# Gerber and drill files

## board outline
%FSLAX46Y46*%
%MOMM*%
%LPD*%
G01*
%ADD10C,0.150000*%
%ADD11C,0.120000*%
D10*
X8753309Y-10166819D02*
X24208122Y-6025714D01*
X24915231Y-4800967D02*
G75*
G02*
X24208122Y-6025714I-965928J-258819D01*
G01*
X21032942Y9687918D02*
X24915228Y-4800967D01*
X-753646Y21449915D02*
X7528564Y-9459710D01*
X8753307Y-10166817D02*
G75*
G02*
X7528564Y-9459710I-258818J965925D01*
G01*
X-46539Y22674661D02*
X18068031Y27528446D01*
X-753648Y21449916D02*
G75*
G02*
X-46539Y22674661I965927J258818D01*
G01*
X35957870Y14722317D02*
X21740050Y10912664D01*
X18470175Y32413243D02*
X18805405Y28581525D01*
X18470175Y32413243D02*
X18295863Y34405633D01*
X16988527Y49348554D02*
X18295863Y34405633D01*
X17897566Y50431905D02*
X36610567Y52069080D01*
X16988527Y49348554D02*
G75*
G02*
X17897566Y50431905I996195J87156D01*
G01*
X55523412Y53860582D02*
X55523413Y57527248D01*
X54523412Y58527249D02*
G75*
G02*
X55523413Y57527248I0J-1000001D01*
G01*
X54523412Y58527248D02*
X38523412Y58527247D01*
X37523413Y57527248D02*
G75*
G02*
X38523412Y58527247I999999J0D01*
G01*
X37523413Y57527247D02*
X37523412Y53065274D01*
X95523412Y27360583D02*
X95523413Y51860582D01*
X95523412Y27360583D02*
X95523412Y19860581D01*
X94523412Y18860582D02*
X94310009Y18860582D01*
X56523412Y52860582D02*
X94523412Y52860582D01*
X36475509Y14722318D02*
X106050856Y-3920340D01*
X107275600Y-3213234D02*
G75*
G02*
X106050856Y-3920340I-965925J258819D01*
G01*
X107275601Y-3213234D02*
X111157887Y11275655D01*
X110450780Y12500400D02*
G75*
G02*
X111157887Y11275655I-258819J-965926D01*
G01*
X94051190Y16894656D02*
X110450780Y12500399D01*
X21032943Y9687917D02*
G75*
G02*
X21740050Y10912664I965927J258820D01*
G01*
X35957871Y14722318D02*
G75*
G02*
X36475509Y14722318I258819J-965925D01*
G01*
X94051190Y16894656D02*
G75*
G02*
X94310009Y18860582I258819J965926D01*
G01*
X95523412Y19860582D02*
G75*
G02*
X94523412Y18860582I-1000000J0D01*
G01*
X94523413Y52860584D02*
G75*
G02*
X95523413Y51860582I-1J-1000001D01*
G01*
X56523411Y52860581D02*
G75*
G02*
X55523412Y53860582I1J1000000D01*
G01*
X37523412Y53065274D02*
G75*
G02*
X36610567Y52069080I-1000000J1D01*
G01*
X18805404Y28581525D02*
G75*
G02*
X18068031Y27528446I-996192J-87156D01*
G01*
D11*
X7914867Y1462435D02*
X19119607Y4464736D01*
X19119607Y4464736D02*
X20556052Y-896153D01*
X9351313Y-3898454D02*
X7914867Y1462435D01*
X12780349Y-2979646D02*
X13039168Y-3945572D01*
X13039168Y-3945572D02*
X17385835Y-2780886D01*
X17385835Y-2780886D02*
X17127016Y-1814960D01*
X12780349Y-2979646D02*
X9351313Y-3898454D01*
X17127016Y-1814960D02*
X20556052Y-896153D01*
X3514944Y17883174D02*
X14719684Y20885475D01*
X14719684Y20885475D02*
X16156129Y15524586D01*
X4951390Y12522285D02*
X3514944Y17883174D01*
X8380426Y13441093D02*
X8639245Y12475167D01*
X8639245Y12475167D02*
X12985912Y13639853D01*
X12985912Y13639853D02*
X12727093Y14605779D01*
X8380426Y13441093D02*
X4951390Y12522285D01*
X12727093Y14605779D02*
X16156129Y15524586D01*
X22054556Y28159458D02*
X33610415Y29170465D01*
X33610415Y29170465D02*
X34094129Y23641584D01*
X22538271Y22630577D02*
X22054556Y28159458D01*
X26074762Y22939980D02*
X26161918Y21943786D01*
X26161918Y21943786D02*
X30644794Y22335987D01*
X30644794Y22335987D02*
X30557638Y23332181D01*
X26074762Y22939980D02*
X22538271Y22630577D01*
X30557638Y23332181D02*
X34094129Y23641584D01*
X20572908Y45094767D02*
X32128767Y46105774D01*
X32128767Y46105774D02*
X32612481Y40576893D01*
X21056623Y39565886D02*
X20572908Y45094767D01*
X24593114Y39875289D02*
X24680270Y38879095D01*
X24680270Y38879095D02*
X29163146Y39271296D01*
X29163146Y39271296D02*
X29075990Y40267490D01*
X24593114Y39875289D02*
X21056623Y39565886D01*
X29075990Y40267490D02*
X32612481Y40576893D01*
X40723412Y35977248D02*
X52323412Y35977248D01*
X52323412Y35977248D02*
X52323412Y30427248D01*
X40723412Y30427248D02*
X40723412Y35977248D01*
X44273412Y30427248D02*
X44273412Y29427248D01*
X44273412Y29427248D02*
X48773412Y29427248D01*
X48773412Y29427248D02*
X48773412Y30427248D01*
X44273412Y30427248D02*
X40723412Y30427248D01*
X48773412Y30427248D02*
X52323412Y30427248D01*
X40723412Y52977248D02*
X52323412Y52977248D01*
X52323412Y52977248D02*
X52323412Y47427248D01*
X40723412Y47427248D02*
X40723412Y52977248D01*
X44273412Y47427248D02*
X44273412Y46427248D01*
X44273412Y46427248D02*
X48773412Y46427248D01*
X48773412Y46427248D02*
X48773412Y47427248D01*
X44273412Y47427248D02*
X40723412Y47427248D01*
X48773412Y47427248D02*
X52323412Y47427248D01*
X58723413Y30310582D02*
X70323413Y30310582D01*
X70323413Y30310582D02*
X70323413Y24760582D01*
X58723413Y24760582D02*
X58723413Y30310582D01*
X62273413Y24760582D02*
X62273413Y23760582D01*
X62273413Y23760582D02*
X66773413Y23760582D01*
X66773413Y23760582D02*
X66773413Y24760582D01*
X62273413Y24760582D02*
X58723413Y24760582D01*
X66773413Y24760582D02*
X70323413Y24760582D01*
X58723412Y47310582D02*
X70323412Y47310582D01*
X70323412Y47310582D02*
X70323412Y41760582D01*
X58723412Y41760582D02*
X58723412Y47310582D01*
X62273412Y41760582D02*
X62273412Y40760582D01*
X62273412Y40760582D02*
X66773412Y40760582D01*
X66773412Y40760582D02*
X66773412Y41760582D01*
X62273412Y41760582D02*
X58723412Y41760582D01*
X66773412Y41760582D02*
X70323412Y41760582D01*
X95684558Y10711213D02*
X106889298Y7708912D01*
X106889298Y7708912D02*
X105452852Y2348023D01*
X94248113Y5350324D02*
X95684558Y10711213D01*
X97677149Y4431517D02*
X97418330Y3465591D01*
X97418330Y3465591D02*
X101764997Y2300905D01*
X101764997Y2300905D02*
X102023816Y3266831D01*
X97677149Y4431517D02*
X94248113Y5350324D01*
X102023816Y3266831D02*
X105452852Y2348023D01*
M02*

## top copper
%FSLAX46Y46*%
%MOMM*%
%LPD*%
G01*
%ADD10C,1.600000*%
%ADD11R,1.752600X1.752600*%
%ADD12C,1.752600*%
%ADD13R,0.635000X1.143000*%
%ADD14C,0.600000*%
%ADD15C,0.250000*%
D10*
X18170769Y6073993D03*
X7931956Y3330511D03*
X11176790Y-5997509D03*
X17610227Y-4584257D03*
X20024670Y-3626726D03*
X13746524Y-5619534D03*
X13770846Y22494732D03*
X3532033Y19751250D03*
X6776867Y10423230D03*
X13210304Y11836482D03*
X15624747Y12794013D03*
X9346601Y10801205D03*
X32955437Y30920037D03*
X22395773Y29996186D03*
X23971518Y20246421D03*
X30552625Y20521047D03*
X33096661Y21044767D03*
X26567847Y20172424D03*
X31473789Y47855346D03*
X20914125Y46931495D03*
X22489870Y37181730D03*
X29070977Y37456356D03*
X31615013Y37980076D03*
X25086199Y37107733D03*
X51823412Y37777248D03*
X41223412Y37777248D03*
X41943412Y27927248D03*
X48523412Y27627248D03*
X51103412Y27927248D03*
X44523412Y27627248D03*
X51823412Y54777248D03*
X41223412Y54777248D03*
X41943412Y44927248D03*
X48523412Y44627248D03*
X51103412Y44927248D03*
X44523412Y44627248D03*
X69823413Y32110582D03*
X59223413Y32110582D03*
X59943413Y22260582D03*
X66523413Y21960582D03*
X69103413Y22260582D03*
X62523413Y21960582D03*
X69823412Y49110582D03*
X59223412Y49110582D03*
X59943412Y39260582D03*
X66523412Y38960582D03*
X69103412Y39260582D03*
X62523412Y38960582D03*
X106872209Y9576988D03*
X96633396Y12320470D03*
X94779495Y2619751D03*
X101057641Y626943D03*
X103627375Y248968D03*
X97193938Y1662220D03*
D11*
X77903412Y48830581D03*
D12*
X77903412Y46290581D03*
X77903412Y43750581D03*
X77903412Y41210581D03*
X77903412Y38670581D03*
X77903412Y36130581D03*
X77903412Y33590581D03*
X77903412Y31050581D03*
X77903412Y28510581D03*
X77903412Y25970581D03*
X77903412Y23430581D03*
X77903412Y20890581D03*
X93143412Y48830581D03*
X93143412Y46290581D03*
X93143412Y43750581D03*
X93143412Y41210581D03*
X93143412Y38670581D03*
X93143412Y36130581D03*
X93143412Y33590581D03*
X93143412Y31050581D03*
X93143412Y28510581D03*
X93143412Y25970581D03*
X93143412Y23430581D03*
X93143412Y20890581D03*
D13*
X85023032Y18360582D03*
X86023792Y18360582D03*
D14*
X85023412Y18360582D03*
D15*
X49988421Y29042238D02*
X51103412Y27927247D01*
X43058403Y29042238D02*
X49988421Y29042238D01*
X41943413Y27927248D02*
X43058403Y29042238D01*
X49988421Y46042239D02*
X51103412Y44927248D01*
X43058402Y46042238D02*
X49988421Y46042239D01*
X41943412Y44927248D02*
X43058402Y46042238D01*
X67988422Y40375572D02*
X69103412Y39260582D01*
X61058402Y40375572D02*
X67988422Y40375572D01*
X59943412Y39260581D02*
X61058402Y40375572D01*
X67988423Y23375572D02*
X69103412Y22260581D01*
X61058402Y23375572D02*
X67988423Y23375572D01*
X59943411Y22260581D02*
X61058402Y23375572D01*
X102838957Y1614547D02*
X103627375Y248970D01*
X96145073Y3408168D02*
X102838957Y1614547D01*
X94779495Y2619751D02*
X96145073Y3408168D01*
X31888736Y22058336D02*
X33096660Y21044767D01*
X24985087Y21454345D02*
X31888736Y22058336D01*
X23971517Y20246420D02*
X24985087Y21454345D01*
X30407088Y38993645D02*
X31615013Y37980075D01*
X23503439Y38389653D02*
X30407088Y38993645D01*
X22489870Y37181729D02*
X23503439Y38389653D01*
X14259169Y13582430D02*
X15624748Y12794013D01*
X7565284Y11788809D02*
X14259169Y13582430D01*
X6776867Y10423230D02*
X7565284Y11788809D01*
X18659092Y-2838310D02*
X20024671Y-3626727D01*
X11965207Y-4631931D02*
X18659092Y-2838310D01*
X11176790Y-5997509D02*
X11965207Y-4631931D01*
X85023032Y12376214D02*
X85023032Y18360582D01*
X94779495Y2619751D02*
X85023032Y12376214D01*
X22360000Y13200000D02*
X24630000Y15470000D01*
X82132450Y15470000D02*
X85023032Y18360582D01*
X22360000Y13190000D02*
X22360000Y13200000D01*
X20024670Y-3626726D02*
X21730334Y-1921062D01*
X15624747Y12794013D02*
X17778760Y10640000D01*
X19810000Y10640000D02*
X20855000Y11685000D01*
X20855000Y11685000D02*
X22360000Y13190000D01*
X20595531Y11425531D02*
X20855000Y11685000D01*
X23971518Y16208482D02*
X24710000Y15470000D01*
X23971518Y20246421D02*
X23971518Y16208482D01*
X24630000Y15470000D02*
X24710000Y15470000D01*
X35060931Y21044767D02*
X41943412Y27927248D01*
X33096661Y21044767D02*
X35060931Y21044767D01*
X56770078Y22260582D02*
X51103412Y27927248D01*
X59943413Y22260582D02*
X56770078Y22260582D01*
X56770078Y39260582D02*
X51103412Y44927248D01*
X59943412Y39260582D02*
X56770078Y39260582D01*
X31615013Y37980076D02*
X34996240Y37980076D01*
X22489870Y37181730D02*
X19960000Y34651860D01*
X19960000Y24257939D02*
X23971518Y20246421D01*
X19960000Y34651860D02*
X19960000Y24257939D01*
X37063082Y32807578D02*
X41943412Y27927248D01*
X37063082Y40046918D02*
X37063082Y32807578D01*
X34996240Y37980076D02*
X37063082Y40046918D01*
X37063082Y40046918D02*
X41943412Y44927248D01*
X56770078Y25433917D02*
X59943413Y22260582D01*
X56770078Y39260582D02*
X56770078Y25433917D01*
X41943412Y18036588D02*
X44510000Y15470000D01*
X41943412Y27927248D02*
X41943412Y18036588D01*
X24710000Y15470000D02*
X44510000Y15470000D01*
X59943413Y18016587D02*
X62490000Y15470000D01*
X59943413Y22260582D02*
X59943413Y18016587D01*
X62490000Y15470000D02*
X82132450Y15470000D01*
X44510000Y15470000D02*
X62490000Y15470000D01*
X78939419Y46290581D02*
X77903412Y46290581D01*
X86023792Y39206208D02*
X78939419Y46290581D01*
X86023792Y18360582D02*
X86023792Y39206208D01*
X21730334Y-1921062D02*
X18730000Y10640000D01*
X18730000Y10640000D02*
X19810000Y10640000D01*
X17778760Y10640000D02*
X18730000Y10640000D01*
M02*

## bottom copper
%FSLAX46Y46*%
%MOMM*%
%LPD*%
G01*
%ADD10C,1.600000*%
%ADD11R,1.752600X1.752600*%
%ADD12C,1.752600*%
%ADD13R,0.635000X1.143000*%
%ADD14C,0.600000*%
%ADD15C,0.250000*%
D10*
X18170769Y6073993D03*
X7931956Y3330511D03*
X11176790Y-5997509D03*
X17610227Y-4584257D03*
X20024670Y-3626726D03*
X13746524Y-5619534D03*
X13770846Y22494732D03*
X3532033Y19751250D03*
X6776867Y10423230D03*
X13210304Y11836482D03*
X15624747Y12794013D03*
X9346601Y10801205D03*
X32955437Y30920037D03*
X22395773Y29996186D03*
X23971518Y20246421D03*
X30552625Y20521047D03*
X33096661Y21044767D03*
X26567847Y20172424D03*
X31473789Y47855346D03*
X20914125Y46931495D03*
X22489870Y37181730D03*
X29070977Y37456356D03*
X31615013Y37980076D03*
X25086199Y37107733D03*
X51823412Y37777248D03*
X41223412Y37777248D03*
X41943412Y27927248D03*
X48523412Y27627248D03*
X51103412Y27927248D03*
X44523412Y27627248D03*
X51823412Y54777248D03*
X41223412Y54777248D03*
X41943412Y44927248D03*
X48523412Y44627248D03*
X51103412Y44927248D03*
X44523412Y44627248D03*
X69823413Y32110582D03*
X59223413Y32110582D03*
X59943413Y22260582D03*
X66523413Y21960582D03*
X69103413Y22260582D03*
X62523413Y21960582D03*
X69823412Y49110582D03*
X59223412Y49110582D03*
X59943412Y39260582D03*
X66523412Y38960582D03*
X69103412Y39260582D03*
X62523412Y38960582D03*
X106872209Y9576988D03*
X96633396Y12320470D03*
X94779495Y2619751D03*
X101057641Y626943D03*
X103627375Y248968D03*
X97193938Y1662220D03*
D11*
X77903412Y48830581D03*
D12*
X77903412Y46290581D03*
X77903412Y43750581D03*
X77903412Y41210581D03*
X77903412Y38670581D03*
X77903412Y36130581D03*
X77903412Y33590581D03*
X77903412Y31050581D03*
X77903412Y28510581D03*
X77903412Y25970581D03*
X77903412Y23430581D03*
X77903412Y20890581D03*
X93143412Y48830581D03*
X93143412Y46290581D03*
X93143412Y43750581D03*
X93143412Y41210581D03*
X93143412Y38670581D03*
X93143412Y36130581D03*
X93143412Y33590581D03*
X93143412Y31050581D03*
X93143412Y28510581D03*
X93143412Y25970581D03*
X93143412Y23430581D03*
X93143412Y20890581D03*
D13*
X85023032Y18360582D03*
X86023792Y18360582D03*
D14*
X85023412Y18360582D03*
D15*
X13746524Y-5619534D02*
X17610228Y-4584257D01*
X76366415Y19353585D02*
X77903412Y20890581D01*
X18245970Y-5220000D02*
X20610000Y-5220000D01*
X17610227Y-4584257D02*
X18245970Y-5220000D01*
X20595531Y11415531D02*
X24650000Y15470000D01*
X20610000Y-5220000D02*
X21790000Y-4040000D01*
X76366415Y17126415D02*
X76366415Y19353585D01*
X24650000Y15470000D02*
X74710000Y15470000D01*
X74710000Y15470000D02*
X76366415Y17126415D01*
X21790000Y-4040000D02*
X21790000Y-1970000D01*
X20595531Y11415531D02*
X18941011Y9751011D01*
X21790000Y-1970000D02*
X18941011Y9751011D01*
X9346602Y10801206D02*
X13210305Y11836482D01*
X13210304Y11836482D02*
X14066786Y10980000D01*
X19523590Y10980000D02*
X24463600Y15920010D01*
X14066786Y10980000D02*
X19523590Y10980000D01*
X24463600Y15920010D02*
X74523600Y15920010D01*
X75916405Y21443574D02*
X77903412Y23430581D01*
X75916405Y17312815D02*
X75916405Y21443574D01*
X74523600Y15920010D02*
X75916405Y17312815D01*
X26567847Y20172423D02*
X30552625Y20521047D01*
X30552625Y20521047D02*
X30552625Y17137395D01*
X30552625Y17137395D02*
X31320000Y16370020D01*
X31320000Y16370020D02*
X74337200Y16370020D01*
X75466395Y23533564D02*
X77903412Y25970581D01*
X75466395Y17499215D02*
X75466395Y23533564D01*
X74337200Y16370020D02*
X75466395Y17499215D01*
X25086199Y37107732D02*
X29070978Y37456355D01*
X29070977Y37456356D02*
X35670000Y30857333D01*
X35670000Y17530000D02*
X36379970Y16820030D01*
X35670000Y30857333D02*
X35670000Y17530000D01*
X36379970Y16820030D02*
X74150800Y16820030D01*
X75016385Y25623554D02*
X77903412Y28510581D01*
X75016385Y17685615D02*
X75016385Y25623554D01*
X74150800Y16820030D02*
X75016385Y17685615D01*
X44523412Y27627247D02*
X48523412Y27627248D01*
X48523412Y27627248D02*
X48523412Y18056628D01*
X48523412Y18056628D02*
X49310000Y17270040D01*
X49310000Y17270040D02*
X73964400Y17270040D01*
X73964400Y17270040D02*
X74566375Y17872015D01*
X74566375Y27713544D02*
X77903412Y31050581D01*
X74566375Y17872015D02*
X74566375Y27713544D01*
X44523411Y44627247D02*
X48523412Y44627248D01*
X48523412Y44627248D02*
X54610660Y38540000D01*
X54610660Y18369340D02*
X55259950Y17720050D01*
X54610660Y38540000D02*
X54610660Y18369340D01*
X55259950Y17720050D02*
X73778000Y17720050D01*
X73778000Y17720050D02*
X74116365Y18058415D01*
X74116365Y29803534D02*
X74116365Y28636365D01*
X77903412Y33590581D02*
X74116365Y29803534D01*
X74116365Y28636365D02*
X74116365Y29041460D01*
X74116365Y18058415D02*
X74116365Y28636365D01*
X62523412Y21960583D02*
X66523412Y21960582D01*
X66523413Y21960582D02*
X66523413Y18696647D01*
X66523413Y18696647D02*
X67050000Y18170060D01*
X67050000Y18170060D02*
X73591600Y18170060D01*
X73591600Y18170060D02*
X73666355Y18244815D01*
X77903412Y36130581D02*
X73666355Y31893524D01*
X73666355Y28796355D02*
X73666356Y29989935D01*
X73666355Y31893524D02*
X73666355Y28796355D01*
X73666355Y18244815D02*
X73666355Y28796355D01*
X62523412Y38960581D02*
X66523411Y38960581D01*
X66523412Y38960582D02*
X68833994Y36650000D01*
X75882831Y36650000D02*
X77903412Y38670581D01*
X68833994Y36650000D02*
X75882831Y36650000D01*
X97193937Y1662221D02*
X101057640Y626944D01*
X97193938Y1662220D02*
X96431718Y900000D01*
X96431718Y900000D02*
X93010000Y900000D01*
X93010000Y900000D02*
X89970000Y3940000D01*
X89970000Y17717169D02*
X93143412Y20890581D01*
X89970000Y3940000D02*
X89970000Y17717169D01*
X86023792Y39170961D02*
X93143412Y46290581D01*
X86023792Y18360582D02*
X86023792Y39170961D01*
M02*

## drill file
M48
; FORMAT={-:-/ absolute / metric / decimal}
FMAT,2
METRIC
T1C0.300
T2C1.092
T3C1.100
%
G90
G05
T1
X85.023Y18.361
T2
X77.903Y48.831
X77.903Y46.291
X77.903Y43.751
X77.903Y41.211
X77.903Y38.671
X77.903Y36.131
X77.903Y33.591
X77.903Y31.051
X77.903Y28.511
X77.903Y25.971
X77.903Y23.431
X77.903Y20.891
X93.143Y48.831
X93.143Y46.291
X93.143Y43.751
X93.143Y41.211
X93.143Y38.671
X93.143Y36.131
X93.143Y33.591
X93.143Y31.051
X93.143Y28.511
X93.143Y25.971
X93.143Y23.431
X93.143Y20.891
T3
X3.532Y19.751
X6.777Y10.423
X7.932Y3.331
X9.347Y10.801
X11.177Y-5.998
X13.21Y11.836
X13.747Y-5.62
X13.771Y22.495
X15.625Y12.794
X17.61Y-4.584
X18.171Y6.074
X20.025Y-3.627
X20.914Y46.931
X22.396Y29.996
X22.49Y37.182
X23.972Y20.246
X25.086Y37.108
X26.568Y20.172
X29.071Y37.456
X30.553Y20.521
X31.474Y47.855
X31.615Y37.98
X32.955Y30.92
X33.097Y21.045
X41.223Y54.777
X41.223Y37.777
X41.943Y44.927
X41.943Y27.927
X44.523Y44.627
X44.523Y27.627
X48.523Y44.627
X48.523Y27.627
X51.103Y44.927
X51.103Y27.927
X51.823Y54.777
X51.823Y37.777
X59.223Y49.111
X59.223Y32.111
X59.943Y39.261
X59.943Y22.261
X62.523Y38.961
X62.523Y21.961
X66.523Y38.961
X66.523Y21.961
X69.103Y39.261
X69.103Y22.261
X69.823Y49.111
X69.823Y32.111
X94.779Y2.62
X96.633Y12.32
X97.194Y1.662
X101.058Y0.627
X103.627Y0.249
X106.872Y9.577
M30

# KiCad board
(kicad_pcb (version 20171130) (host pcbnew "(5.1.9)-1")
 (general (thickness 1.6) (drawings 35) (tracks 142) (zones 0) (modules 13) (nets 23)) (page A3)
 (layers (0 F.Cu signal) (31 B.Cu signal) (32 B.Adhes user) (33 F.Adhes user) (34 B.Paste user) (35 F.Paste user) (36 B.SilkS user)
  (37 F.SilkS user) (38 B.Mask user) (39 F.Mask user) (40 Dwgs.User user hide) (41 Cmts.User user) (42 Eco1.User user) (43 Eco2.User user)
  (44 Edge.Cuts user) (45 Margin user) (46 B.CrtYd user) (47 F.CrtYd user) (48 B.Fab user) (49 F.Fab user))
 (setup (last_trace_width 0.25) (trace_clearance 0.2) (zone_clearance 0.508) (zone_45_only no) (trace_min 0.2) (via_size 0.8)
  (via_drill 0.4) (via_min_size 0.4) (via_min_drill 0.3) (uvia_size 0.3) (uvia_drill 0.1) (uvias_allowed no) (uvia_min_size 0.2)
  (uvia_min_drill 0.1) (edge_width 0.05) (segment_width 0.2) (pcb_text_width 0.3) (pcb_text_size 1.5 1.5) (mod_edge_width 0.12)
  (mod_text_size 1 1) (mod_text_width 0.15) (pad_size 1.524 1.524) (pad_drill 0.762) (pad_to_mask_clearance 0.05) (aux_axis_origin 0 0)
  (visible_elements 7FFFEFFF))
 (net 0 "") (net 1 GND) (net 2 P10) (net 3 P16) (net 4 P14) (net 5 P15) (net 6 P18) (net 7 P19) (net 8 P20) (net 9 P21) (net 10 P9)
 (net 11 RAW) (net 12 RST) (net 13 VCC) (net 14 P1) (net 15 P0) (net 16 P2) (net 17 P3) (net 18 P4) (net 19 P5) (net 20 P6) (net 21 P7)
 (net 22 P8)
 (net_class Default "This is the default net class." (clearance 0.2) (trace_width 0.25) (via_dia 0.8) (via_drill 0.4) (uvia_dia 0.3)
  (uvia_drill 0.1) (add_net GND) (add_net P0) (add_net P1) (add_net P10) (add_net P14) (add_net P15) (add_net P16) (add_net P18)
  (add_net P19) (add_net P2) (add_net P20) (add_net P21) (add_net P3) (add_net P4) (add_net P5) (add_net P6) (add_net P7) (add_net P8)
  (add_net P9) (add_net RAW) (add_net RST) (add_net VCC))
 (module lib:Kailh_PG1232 (layer F.Cu) (at 14.280753 -0.114104 15)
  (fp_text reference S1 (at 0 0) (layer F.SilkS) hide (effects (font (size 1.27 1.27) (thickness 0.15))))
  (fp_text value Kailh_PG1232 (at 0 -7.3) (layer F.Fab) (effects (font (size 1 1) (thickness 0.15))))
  (fp_line (start -5.8 -2.95) (end 5.8 -2.95) (layer Edge.Cuts) (width 0.12))
  (fp_line (start 5.8 -2.95) (end 5.8 2.6) (layer Edge.Cuts) (width 0.12))
  (fp_line (start -5.8 2.6) (end -5.8 -2.95) (layer Edge.Cuts) (width 0.12))
  (fp_line (start -2.25 2.6) (end -2.25 3.6) (layer Edge.Cuts) (width 0.12))
  (fp_line (start -2.25 3.6) (end 2.25 3.6) (layer Edge.Cuts) (width 0.12))
  (fp_line (start 2.25 3.6) (end 2.25 2.6) (layer Edge.Cuts) (width 0.12))
  (fp_line (start -2.25 2.6) (end -5.8 2.6) (layer Edge.Cuts) (width 0.12))
  (fp_line (start 2.25 2.6) (end 5.8 2.6) (layer Edge.Cuts) (width 0.12))
  (pad 3 thru_hole circle (at 5.3 -4.75) (size 1.6 1.6) (drill 1.1) (layers *.Cu *.Mask) (clearance 0.2))
  (pad 4 thru_hole circle (at -5.3 -4.75) (size 1.6 1.6) (drill 1.1) (layers *.Cu *.Mask) (clearance 0.2))
  (pad 1 thru_hole circle (at -4.58 5.1) (size 1.6 1.6) (drill 1.1) (layers *.Cu *.Mask) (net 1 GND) (clearance 0.2))
  (pad 2 thru_hole circle (at 2 5.4) (size 1.6 1.6) (drill 1.1) (layers *.Cu *.Mask) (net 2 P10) (clearance 0.2))
  (pad 1 thru_hole circle (at 4.58 5.1) (size 1.6 1.6) (drill 1.1) (layers *.Cu *.Mask) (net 1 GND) (clearance 0.2))
  (pad 2 thru_hole circle (at -2 5.4) (size 1.6 1.6) (drill 1.1) (layers *.Cu *.Mask) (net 2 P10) (clearance 0.2)))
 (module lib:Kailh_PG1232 (layer F.Cu) (at 9.88083 -16.534843 15)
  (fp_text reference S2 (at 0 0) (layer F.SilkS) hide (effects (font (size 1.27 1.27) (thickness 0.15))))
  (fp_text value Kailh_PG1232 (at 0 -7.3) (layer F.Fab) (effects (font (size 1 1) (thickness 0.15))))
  (fp_line (start -5.8 -2.95) (end 5.8 -2.95) (layer Edge.Cuts) (width 0.12))
  (fp_line (start 5.8 -2.95) (end 5.8 2.6) (layer Edge.Cuts) (width 0.12))
  (fp_line (start -5.8 2.6) (end -5.8 -2.95) (layer Edge.Cuts) (width 0.12))
  (fp_line (start -2.25 2.6) (end -2.25 3.6) (layer Edge.Cuts) (width 0.12))
  (fp_line (start -2.25 3.6) (end 2.25 3.6) (layer Edge.Cuts) (width 0.12))
  (fp_line (start 2.25 3.6) (end 2.25 2.6) (layer Edge.Cuts) (width 0.12))
  (fp_line (start -2.25 2.6) (end -5.8 2.6) (layer Edge.Cuts) (width 0.12))
  (fp_line (start 2.25 2.6) (end 5.8 2.6) (layer Edge.Cuts) (width 0.12))
  (pad 3 thru_hole circle (at 5.3 -4.75) (size 1.6 1.6) (drill 1.1) (layers *.Cu *.Mask) (clearance 0.2))
  (pad 4 thru_hole circle (at -5.3 -4.75) (size 1.6 1.6) (drill 1.1) (layers *.Cu *.Mask) (clearance 0.2))
  (pad 1 thru_hole circle (at -4.58 5.1) (size 1.6 1.6) (drill 1.1) (layers *.Cu *.Mask) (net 1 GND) (clearance 0.2))
  (pad 2 thru_hole circle (at 2 5.4) (size 1.6 1.6) (drill 1.1) (layers *.Cu *.Mask) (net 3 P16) (clearance 0.2))
  (pad 1 thru_hole circle (at 4.58 5.1) (size 1.6 1.6) (drill 1.1) (layers *.Cu *.Mask) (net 1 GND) (clearance 0.2))
  (pad 2 thru_hole circle (at -2 5.4) (size 1.6 1.6) (drill 1.1) (layers *.Cu *.Mask) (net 3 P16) (clearance 0.2)))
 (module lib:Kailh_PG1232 (layer F.Cu) (at 28.089595 -25.726187 5)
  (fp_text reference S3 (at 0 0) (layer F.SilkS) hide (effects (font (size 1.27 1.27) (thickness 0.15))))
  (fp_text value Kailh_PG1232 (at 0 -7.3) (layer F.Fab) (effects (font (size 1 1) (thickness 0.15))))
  (fp_line (start -5.8 -2.95) (end 5.8 -2.95) (layer Edge.Cuts) (width 0.12))
  (fp_line (start 5.8 -2.95) (end 5.8 2.6) (layer Edge.Cuts) (width 0.12))
  (fp_line (start -5.8 2.6) (end -5.8 -2.95) (layer Edge.Cuts) (width 0.12))
  (fp_line (start -2.25 2.6) (end -2.25 3.6) (layer Edge.Cuts) (width 0.12))
  (fp_line (start -2.25 3.6) (end 2.25 3.6) (layer Edge.Cuts) (width 0.12))
  (fp_line (start 2.25 3.6) (end 2.25 2.6) (layer Edge.Cuts) (width 0.12))
  (fp_line (start -2.25 2.6) (end -5.8 2.6) (layer Edge.Cuts) (width 0.12))
  (fp_line (start 2.25 2.6) (end 5.8 2.6) (layer Edge.Cuts) (width 0.12))
  (pad 3 thru_hole circle (at 5.3 -4.75) (size 1.6 1.6) (drill 1.1) (layers *.Cu *.Mask) (clearance 0.2))
  (pad 4 thru_hole circle (at -5.3 -4.75) (size 1.6 1.6) (drill 1.1) (layers *.Cu *.Mask) (clearance 0.2))
  (pad 1 thru_hole circle (at -4.58 5.1) (size 1.6 1.6) (drill 1.1) (layers *.Cu *.Mask) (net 1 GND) (clearance 0.2))
  (pad 2 thru_hole circle (at 2 5.4) (size 1.6 1.6) (drill 1.1) (layers *.Cu *.Mask) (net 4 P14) (clearance 0.2))
  (pad 1 thru_hole circle (at 4.58 5.1) (size 1.6 1.6) (drill 1.1) (layers *.Cu *.Mask) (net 1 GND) (clearance 0.2))
  (pad 2 thru_hole circle (at -2 5.4) (size 1.6 1.6) (drill 1.1) (layers *.Cu *.Mask) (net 4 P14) (clearance 0.2)))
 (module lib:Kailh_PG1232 (layer F.Cu) (at 26.607947 -42.661496 5)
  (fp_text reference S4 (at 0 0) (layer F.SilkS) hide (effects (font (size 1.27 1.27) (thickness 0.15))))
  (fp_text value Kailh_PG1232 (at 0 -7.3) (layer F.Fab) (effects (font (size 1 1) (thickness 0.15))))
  (fp_line (start -5.8 -2.95) (end 5.8 -2.95) (layer Edge.Cuts) (width 0.12))
  (fp_line (start 5.8 -2.95) (end 5.8 2.6) (layer Edge.Cuts) (width 0.12))
  (fp_line (start -5.8 2.6) (end -5.8 -2.95) (layer Edge.Cuts) (width 0.12))
  (fp_line (start -2.25 2.6) (end -2.25 3.6) (layer Edge.Cuts) (width 0.12))
  (fp_line (start -2.25 3.6) (end 2.25 3.6) (layer Edge.Cuts) (width 0.12))
  (fp_line (start 2.25 3.6) (end 2.25 2.6) (layer Edge.Cuts) (width 0.12))
  (fp_line (start -2.25 2.6) (end -5.8 2.6) (layer Edge.Cuts) (width 0.12))
  (fp_line (start 2.25 2.6) (end 5.8 2.6) (layer Edge.Cuts) (width 0.12))
  (pad 3 thru_hole circle (at 5.3 -4.75) (size 1.6 1.6) (drill 1.1) (layers *.Cu *.Mask) (clearance 0.2))
  (pad 4 thru_hole circle (at -5.3 -4.75) (size 1.6 1.6) (drill 1.1) (layers *.Cu *.Mask) (clearance 0.2))
  (pad 1 thru_hole circle (at -4.58 5.1) (size 1.6 1.6) (drill 1.1) (layers *.Cu *.Mask) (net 1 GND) (clearance 0.2))
  (pad 2 thru_hole circle (at 2 5.4) (size 1.6 1.6) (drill 1.1) (layers *.Cu *.Mask) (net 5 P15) (clearance 0.2))
  (pad 1 thru_hole circle (at 4.58 5.1) (size 1.6 1.6) (drill 1.1) (layers *.Cu *.Mask) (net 1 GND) (clearance 0.2))
  (pad 2 thru_hole circle (at -2 5.4) (size 1.6 1.6) (drill 1.1) (layers *.Cu *.Mask) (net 5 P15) (clearance 0.2)))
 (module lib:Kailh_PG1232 (layer F.Cu) (at 46.523412 -33.027248)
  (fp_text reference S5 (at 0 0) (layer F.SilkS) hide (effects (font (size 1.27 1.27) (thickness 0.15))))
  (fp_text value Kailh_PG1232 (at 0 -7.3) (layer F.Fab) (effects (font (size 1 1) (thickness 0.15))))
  (fp_line (start -5.8 -2.95) (end 5.8 -2.95) (layer Edge.Cuts) (width 0.12))
  (fp_line (start 5.8 -2.95) (end 5.8 2.6) (layer Edge.Cuts) (width 0.12))
  (fp_line (start -5.8 2.6) (end -5.8 -2.95) (layer Edge.Cuts) (width 0.12))
  (fp_line (start -2.25 2.6) (end -2.25 3.6) (layer Edge.Cuts) (width 0.12))
  (fp_line (start -2.25 3.6) (end 2.25 3.6) (layer Edge.Cuts) (width 0.12))
  (fp_line (start 2.25 3.6) (end 2.25 2.6) (layer Edge.Cuts) (width 0.12))
  (fp_line (start -2.25 2.6) (end -5.8 2.6) (layer Edge.Cuts) (width 0.12))
  (fp_line (start 2.25 2.6) (end 5.8 2.6) (layer Edge.Cuts) (width 0.12))
  (pad 3 thru_hole circle (at 5.3 -4.75) (size 1.6 1.6) (drill 1.1) (layers *.Cu *.Mask) (clearance 0.2))
  (pad 4 thru_hole circle (at -5.3 -4.75) (size 1.6 1.6) (drill 1.1) (layers *.Cu *.Mask) (clearance 0.2))
  (pad 1 thru_hole circle (at -4.58 5.1) (size 1.6 1.6) (drill 1.1) (layers *.Cu *.Mask) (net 1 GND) (clearance 0.2))
  (pad 2 thru_hole circle (at 2 5.4) (size 1.6 1.6) (drill 1.1) (layers *.Cu *.Mask) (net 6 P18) (clearance 0.2))
  (pad 1 thru_hole circle (at 4.58 5.1) (size 1.6 1.6) (drill 1.1) (layers *.Cu *.Mask) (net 1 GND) (clearance 0.2))
  (pad 2 thru_hole circle (at -2 5.4) (size 1.6 1.6) (drill 1.1) (layers *.Cu *.Mask) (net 6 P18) (clearance 0.2)))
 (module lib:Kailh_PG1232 (layer F.Cu) (at 46.523412 -50.027248)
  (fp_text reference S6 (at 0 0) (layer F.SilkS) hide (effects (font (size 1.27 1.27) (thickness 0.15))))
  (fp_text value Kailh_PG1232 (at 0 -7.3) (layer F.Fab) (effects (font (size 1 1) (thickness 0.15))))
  (fp_line (start -5.8 -2.95) (end 5.8 -2.95) (layer Edge.Cuts) (width 0.12))
  (fp_line (start 5.8 -2.95) (end 5.8 2.6) (layer Edge.Cuts) (width 0.12))
  (fp_line (start -5.8 2.6) (end -5.8 -2.95) (layer Edge.Cuts) (width 0.12))
  (fp_line (start -2.25 2.6) (end -2.25 3.6) (layer Edge.Cuts) (width 0.12))
  (fp_line (start -2.25 3.6) (end 2.25 3.6) (layer Edge.Cuts) (width 0.12))
  (fp_line (start 2.25 3.6) (end 2.25 2.6) (layer Edge.Cuts) (width 0.12))
  (fp_line (start -2.25 2.6) (end -5.8 2.6) (layer Edge.Cuts) (width 0.12))
  (fp_line (start 2.25 2.6) (end 5.8 2.6) (layer Edge.Cuts) (width 0.12))
  (pad 3 thru_hole circle (at 5.3 -4.75) (size 1.6 1.6) (drill 1.1) (layers *.Cu *.Mask) (clearance 0.2))
  (pad 4 thru_hole circle (at -5.3 -4.75) (size 1.6 1.6) (drill 1.1) (layers *.Cu *.Mask) (clearance 0.2))
  (pad 1 thru_hole circle (at -4.58 5.1) (size 1.6 1.6) (drill 1.1) (layers *.Cu *.Mask) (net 1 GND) (clearance 0.2))
  (pad 2 thru_hole circle (at 2 5.4) (size 1.6 1.6) (drill 1.1) (layers *.Cu *.Mask) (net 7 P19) (clearance 0.2))
  (pad 1 thru_hole circle (at 4.58 5.1) (size 1.6 1.6) (drill 1.1) (layers *.Cu *.Mask) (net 1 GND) (clearance 0.2))
  (pad 2 thru_hole circle (at -2 5.4) (size 1.6 1.6) (drill 1.1) (layers *.Cu *.Mask) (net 7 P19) (clearance 0.2)))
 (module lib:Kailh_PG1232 (layer F.Cu) (at 64.523413 -27.360582)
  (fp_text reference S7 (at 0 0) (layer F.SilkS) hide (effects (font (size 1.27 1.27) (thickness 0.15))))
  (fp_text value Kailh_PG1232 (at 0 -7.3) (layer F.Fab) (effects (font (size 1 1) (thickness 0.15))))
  (fp_line (start -5.8 -2.95) (end 5.8 -2.95) (layer Edge.Cuts) (width 0.12))
  (fp_line (start 5.8 -2.95) (end 5.8 2.6) (layer Edge.Cuts) (width 0.12))
  (fp_line (start -5.8 2.6) (end -5.8 -2.95) (layer Edge.Cuts) (width 0.12))
  (fp_line (start -2.25 2.6) (end -2.25 3.6) (layer Edge.Cuts) (width 0.12))
  (fp_line (start -2.25 3.6) (end 2.25 3.6) (layer Edge.Cuts) (width 0.12))
  (fp_line (start 2.25 3.6) (end 2.25 2.6) (layer Edge.Cuts) (width 0.12))
  (fp_line (start -2.25 2.6) (end -5.8 2.6) (layer Edge.Cuts) (width 0.12))
  (fp_line (start 2.25 2.6) (end 5.8 2.6) (layer Edge.Cuts) (width 0.12))
  (pad 3 thru_hole circle (at 5.3 -4.75) (size 1.6 1.6) (drill 1.1) (layers *.Cu *.Mask) (clearance 0.2))
  (pad 4 thru_hole circle (at -5.3 -4.75) (size 1.6 1.6) (drill 1.1) (layers *.Cu *.Mask) (clearance 0.2))
  (pad 1 thru_hole circle (at -4.58 5.1) (size 1.6 1.6) (drill 1.1) (layers *.Cu *.Mask) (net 1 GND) (clearance 0.2))
  (pad 2 thru_hole circle (at 2 5.4) (size 1.6 1.6) (drill 1.1) (layers *.Cu *.Mask) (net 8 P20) (clearance 0.2))
  (pad 1 thru_hole circle (at 4.58 5.1) (size 1.6 1.6) (drill 1.1) (layers *.Cu *.Mask) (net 1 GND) (clearance 0.2))
  (pad 2 thru_hole circle (at -2 5.4) (size 1.6 1.6) (drill 1.1) (layers *.Cu *.Mask) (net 8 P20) (clearance 0.2)))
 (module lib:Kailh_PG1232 (layer F.Cu) (at 64.523412 -44.360582)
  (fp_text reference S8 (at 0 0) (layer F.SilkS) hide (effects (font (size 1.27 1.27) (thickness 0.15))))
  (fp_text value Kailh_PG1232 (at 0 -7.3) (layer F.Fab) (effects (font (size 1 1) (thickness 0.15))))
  (fp_line (start -5.8 -2.95) (end 5.8 -2.95) (layer Edge.Cuts) (width 0.12))
  (fp_line (start 5.8 -2.95) (end 5.8 2.6) (layer Edge.Cuts) (width 0.12))
  (fp_line (start -5.8 2.6) (end -5.8 -2.95) (layer Edge.Cuts) (width 0.12))
  (fp_line (start -2.25 2.6) (end -2.25 3.6) (layer Edge.Cuts) (width 0.12))
  (fp_line (start -2.25 3.6) (end 2.25 3.6) (layer Edge.Cuts) (width 0.12))
  (fp_line (start 2.25 3.6) (end 2.25 2.6) (layer Edge.Cuts) (width 0.12))
  (fp_line (start -2.25 2.6) (end -5.8 2.6) (layer Edge.Cuts) (width 0.12))
  (fp_line (start 2.25 2.6) (end 5.8 2.6) (layer Edge.Cuts) (width 0.12))
  (pad 3 thru_hole circle (at 5.3 -4.75) (size 1.6 1.6) (drill 1.1) (layers *.Cu *.Mask) (clearance 0.2))
  (pad 4 thru_hole circle (at -5.3 -4.75) (size 1.6 1.6) (drill 1.1) (layers *.Cu *.Mask) (clearance 0.2))
  (pad 1 thru_hole circle (at -4.58 5.1) (size 1.6 1.6) (drill 1.1) (layers *.Cu *.Mask) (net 1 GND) (clearance 0.2))
  (pad 2 thru_hole circle (at 2 5.4) (size 1.6 1.6) (drill 1.1) (layers *.Cu *.Mask) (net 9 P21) (clearance 0.2))
  (pad 1 thru_hole circle (at 4.58 5.1) (size 1.6 1.6) (drill 1.1) (layers *.Cu *.Mask) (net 1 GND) (clearance 0.2))
  (pad 2 thru_hole circle (at -2 5.4) (size 1.6 1.6) (drill 1.1) (layers *.Cu *.Mask) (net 9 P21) (clearance 0.2)))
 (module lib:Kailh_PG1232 (layer F.Cu) (at 100.523412 -6.360581 345)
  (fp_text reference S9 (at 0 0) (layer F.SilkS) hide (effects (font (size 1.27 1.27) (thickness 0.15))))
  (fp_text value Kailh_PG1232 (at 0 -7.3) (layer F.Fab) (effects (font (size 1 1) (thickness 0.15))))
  (fp_line (start -5.8 -2.95) (end 5.8 -2.95) (layer Edge.Cuts) (width 0.12))
  (fp_line (start 5.8 -2.95) (end 5.8 2.6) (layer Edge.Cuts) (width 0.12))
  (fp_line (start -5.8 2.6) (end -5.8 -2.95) (layer Edge.Cuts) (width 0.12))
  (fp_line (start -2.25 2.6) (end -2.25 3.6) (layer Edge.Cuts) (width 0.12))
  (fp_line (start -2.25 3.6) (end 2.25 3.6) (layer Edge.Cuts) (width 0.12))
  (fp_line (start 2.25 3.6) (end 2.25 2.6) (layer Edge.Cuts) (width 0.12))
  (fp_line (start -2.25 2.6) (end -5.8 2.6) (layer Edge.Cuts) (width 0.12))
  (fp_line (start 2.25 2.6) (end 5.8 2.6) (layer Edge.Cuts) (width 0.12))
  (pad 3 thru_hole circle (at 5.3 -4.75) (size 1.6 1.6) (drill 1.1) (layers *.Cu *.Mask) (clearance 0.2))
  (pad 4 thru_hole circle (at -5.3 -4.75) (size 1.6 1.6) (drill 1.1) (layers *.Cu *.Mask) (clearance 0.2))
  (pad 1 thru_hole circle (at -4.58 5.1) (size 1.6 1.6) (drill 1.1) (layers *.Cu *.Mask) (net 1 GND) (clearance 0.2))
  (pad 2 thru_hole circle (at 2 5.4) (size 1.6 1.6) (drill 1.1) (layers *.Cu *.Mask) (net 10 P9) (clearance 0.2))
  (pad 1 thru_hole circle (at 4.58 5.1) (size 1.6 1.6) (drill 1.1) (layers *.Cu *.Mask) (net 1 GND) (clearance 0.2))
  (pad 2 thru_hole circle (at -2 5.4) (size 1.6 1.6) (drill 1.1) (layers *.Cu *.Mask) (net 10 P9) (clearance 0.2)))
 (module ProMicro (layer F.Cu) (at 85.523412 -34.860581 270)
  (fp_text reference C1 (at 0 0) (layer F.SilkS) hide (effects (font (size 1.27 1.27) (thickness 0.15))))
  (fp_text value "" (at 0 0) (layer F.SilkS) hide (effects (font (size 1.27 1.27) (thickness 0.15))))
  (pad 1 thru_hole rect (at -13.97 7.62 270) (size 1.7526 1.7526) (drill 1.0922) (layers *.Cu *.SilkS *.Mask) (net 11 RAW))
  (pad 2 thru_hole circle (at -11.43 7.62) (size 1.7526 1.7526) (drill 1.0922) (layers *.Cu *.SilkS *.Mask) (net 1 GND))
  (pad 3 thru_hole circle (at -8.89 7.62) (size 1.7526 1.7526) (drill 1.0922) (layers *.Cu *.SilkS *.Mask) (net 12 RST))
  (pad 4 thru_hole circle (at -6.35 7.62) (size 1.7526 1.7526) (drill 1.0922) (layers *.Cu *.SilkS *.Mask) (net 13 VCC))
  (pad 5 thru_hole circle (at -3.81 7.62) (size 1.7526 1.7526) (drill 1.0922) (layers *.Cu *.SilkS *.Mask) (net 9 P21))
  (pad 6 thru_hole circle (at -1.27 7.62) (size 1.7526 1.7526) (drill 1.0922) (layers *.Cu *.SilkS *.Mask) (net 8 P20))
  (pad 7 thru_hole circle (at 1.27 7.62) (size 1.7526 1.7526) (drill 1.0922) (layers *.Cu *.SilkS *.Mask) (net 7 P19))
  (pad 8 thru_hole circle (at 3.81 7.62) (size 1.7526 1.7526) (drill 1.0922) (layers *.Cu *.SilkS *.Mask) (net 6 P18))
  (pad 9 thru_hole circle (at 6.35 7.62) (size 1.7526 1.7526) (drill 1.0922) (layers *.Cu *.SilkS *.Mask) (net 5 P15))
  (pad 10 thru_hole circle (at 8.89 7.62) (size 1.7526 1.7526) (drill 1.0922) (layers *.Cu *.SilkS *.Mask) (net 4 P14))
  (pad 11 thru_hole circle (at 11.43 7.62) (size 1.7526 1.7526) (drill 1.0922) (layers *.Cu *.SilkS *.Mask) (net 3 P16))
  (pad 12 thru_hole circle (at 13.97 7.62) (size 1.7526 1.7526) (drill 1.0922) (layers *.Cu *.SilkS *.Mask) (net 2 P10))
  (pad 13 thru_hole circle (at -13.97 -7.62) (size 1.7526 1.7526) (drill 1.0922) (layers *.Cu *.SilkS *.Mask) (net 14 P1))
  (pad 14 thru_hole circle (at -11.43 -7.62) (size 1.7526 1.7526) (drill 1.0922) (layers *.Cu *.SilkS *.Mask) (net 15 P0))
  (pad 15 thru_hole circle (at -8.89 -7.62) (size 1.7526 1.7526) (drill 1.0922) (layers *.Cu *.SilkS *.Mask) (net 1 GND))
  (pad 16 thru_hole circle (at -6.35 -7.62) (size 1.7526 1.7526) (drill 1.0922) (layers *.Cu *.SilkS *.Mask) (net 1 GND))
  (pad 17 thru_hole circle (at -3.81 -7.62) (size 1.7526 1.7526) (drill 1.0922) (layers *.Cu *.SilkS *.Mask) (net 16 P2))
  (pad 18 thru_hole circle (at -1.27 -7.62) (size 1.7526 1.7526) (drill 1.0922) (layers *.Cu *.SilkS *.Mask) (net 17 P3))
  (pad 19 thru_hole circle (at 1.27 -7.62) (size 1.7526 1.7526) (drill 1.0922) (layers *.Cu *.SilkS *.Mask) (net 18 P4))
  (pad 20 thru_hole circle (at 3.81 -7.62) (size 1.7526 1.7526) (drill 1.0922) (layers *.Cu *.SilkS *.Mask) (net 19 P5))
  (pad 21 thru_hole circle (at 6.35 -7.62) (size 1.7526 1.7526) (drill 1.0922) (layers *.Cu *.SilkS *.Mask) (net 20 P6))
  (pad 22 thru_hole circle (at 8.89 -7.62) (size 1.7526 1.7526) (drill 1.0922) (layers *.Cu *.SilkS *.Mask) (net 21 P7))
  (pad 23 thru_hole circle (at 11.43 -7.62) (size 1.7526 1.7526) (drill 1.0922) (layers *.Cu *.SilkS *.Mask) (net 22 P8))
  (pad 24 thru_hole circle (at 13.97 -7.62) (size 1.7526 1.7526) (drill 1.0922) (layers *.Cu *.SilkS *.Mask) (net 10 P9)))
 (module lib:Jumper (layer F.Cu) (at 85.523412 -18.360582)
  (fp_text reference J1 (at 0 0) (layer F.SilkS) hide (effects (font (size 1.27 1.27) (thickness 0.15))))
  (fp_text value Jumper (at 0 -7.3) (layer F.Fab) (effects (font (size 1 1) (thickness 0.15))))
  (pad 1 smd rect (at -0.50038 0) (size 0.635 1.143) (layers F.Cu F.Paste F.Mask) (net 1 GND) (clearance 0.1905))
  (pad 2 smd rect (at 0.50038 0) (size 0.635 1.143) (layers F.Cu F.Paste F.Mask) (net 1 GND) (clearance 0.1905)))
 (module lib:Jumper (layer F.Cu) (at 85.523412 -18.360582)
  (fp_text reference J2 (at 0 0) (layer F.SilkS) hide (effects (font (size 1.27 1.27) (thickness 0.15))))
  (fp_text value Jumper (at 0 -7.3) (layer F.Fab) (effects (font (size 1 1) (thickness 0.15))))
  (pad 1 smd rect (at -0.50038 0) (size 0.635 1.143) (layers B.Cu B.Paste B.Mask) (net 1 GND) (clearance 0.1905))
  (pad 2 smd rect (at 0.50038 0) (size 0.635 1.143) (layers B.Cu B.Paste B.Mask) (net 15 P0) (clearance 0.1905)))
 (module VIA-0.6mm (layer F.Cu) (at 85.023412 -18.360582)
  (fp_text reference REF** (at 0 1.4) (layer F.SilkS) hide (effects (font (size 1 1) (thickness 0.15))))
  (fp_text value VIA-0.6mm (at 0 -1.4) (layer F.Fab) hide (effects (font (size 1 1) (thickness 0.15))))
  (pad 1 thru_hole circle (at 0 0) (size 0.6 0.6) (drill 0.3) (layers *.Cu) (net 1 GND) (zone_connect 2)))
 (gr_line (start 8.753309 10.166819) (end 24.208122 6.025714) (angle 90) (layer Edge.Cuts) (width 0.15))
 (gr_arc (start 23.949303 5.059786) (end 24.208122 6.025714) (angle -90) (layer Edge.Cuts) (width 0.15))
 (gr_line (start 21.032942 -9.687918) (end 24.915228 4.800967) (angle 90) (layer Edge.Cuts) (width 0.15))
 (gr_line (start -0.753646 -21.449915) (end 7.528564 9.45971) (angle 90) (layer Edge.Cuts) (width 0.15))
 (gr_arc (start 8.494489 9.200892) (end 7.528564 9.45971) (angle -90) (layer Edge.Cuts) (width 0.15))
 (gr_line (start -0.046539 -22.674661) (end 18.068031 -27.528446) (angle 90) (layer Edge.Cuts) (width 0.15))
 (gr_arc (start 0.212279 -21.708734) (end -0.046539 -22.674661) (angle -90) (layer Edge.Cuts) (width 0.15))
 (gr_line (start 35.95787 -14.722317) (end 21.74005 -10.912664) (angle 90) (layer Edge.Cuts) (width 0.15))
 (gr_line (start 18.470175 -32.413243) (end 18.805405 -28.581525) (angle 90) (layer Edge.Cuts) (width 0.15))
 (gr_line (start 18.470175 -32.413243) (end 18.295863 -34.405633) (angle 90) (layer Edge.Cuts) (width 0.15))
 (gr_line (start 16.988527 -49.348554) (end 18.295863 -34.405633) (angle 90) (layer Edge.Cuts) (width 0.15))
 (gr_line (start 17.897566 -50.431905) (end 36.610567 -52.06908) (angle 90) (layer Edge.Cuts) (width 0.15))
 (gr_arc (start 17.984722 -49.43571) (end 17.897566 -50.431905) (angle -90) (layer Edge.Cuts) (width 0.15))
 (gr_line (start 55.523412 -53.860582) (end 55.523413 -57.527248) (angle 90) (layer Edge.Cuts) (width 0.15))
 (gr_arc (start 54.523412 -57.527248) (end 55.523413 -57.527248) (angle -90) (layer Edge.Cuts) (width 0.15))
 (gr_line (start 54.523412 -58.527248) (end 38.523412 -58.527247) (angle 90) (layer Edge.Cuts) (width 0.15))
 (gr_arc (start 38.523412 -57.527248) (end 38.523412 -58.527247) (angle -90) (layer Edge.Cuts) (width 0.15))
 (gr_line (start 37.523413 -57.527247) (end 37.523412 -53.065274) (angle 90) (layer Edge.Cuts) (width 0.15))
 (gr_line (start 95.523412 -27.360583) (end 95.523413 -51.860582) (angle 90) (layer Edge.Cuts) (width 0.15))
 (gr_line (start 95.523412 -27.360583) (end 95.523412 -19.860581) (angle 90) (layer Edge.Cuts) (width 0.15))
 (gr_line (start 94.523412 -18.860582) (end 94.310009 -18.860582) (angle 90) (layer Edge.Cuts) (width 0.15))
 (gr_line (start 56.523412 -52.860582) (end 94.523412 -52.860582) (angle 90) (layer Edge.Cuts) (width 0.15))
 (gr_line (start 36.475509 -14.722318) (end 106.050856 3.92034) (angle 90) (layer Edge.Cuts) (width 0.15))
 (gr_arc (start 106.309675 2.954415) (end 106.050856 3.92034) (angle -90) (layer Edge.Cuts) (width 0.15))
 (gr_line (start 107.275601 3.213234) (end 111.157887 -11.275655) (angle 90) (layer Edge.Cuts) (width 0.15))
 (gr_arc (start 110.191961 -11.534474) (end 111.157887 -11.275655) (angle -90) (layer Edge.Cuts) (width 0.15))
 (gr_line (start 94.05119 -16.894656) (end 110.45078 -12.500399) (angle 90) (layer Edge.Cuts) (width 0.15))
 (gr_arc (start 21.99887 -9.946737) (end 21.74005 -10.912664) (angle -90) (layer Edge.Cuts) (width 0.15))
 (gr_arc (start 36.21669 -13.756393) (end 36.475509 -14.722318) (angle -29.99999579) (layer Edge.Cuts) (width 0.15))
 (gr_arc (start 94.310009 -17.860582) (end 94.310009 -18.860582) (angle -165.0000021) (layer Edge.Cuts) (width 0.15))
 (gr_arc (start 94.523412 -19.860582) (end 94.523412 -18.860582) (angle -90) (layer Edge.Cuts) (width 0.15))
 (gr_arc (start 94.523412 -51.860583) (end 95.523413 -51.860582) (angle -90) (layer Edge.Cuts) (width 0.15))
 (gr_arc (start 56.523412 -53.860581) (end 55.523412 -53.860582) (angle -90) (layer Edge.Cuts) (width 0.15))
 (gr_arc (start 36.523412 -53.065275) (end 36.610567 -52.06908) (angle -85.00000245) (layer Edge.Cuts) (width 0.15))
 (gr_arc (start 17.809212 -28.494369) (end 18.068031 -27.528446) (angle -79.99999966) (layer Edge.Cuts) (width 0.15))
 (segment (start 49.988421 -29.042238) (end 51.103412 -27.927247) (width 0.25) (layer F.Cu) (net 1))
 (segment (start 43.058403 -29.042238) (end 49.988421 -29.042238) (width 0.25) (layer F.Cu) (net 1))
 (segment (start 41.943413 -27.927248) (end 43.058403 -29.042238) (width 0.25) (layer F.Cu) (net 1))
 (segment (start 49.988421 -46.042239) (end 51.103412 -44.927248) (width 0.25) (layer F.Cu) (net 1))
 (segment (start 43.058402 -46.042238) (end 49.988421 -46.042239) (width 0.25) (layer F.Cu) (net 1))
 (segment (start 41.943412 -44.927248) (end 43.058402 -46.042238) (width 0.25) (layer F.Cu) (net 1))
 (segment (start 67.988422 -40.375572) (end 69.103412 -39.260582) (width 0.25) (layer F.Cu) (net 1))
 (segment (start 61.058402 -40.375572) (end 67.988422 -40.375572) (width 0.25) (layer F.Cu) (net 1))
 (segment (start 59.943412 -39.260581) (end 61.058402 -40.375572) (width 0.25) (layer F.Cu) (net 1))
 (segment (start 67.988423 -23.375572) (end 69.103412 -22.260581) (width 0.25) (layer F.Cu) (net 1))
 (segment (start 61.058402 -23.375572) (end 67.988423 -23.375572) (width 0.25) (layer F.Cu) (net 1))
 (segment (start 59.943411 -22.260581) (end 61.058402 -23.375572) (width 0.25) (layer F.Cu) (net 1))
 (segment (start 102.838957 -1.614547) (end 103.627375 -0.24897) (width 0.25) (layer F.Cu) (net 1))
 (segment (start 96.145073 -3.408168) (end 102.838957 -1.614547) (width 0.25) (layer F.Cu) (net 1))
 (segment (start 94.779495 -2.619751) (end 96.145073 -3.408168) (width 0.25) (layer F.Cu) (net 1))
 (segment (start 31.888736 -22.058336) (end 33.09666 -21.044767) (width 0.25) (layer F.Cu) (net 1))
 (segment (start 24.985087 -21.454345) (end 31.888736 -22.058336) (width 0.25) (layer F.Cu) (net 1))
 (segment (start 23.971517 -20.24642) (end 24.985087 -21.454345) (width 0.25) (layer F.Cu) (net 1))
 (segment (start 30.407088 -38.993645) (end 31.615013 -37.980075) (width 0.25) (layer F.Cu) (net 1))
 (segment (start 23.503439 -38.389653) (end 30.407088 -38.993645) (width 0.25) (layer F.Cu) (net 1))
 (segment (start 22.48987 -37.181729) (end 23.503439 -38.389653) (width 0.25) (layer F.Cu) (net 1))
 (segment (start 14.259169 -13.58243) (end 15.624748 -12.794013) (width 0.25) (layer F.Cu) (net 1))
 (segment (start 7.565284 -11.788809) (end 14.259169 -13.58243) (width 0.25) (layer F.Cu) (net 1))
 (segment (start 6.776867 -10.42323) (end 7.565284 -11.788809) (width 0.25) (layer F.Cu) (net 1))
 (segment (start 18.659092 2.83831) (end 20.024671 3.626727) (width 0.25) (layer F.Cu) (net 1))
 (segment (start 11.965207 4.631931) (end 18.659092 2.83831) (width 0.25) (layer F.Cu) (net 1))
 (segment (start 11.17679 5.997509) (end 11.965207 4.631931) (width 0.25) (layer F.Cu) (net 1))
 (segment (start 85.023032 -12.376214) (end 85.023032 -18.360582) (width 0.25) (layer F.Cu) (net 1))
 (segment (start 94.779495 -2.619751) (end 85.023032 -12.376214) (width 0.25) (layer F.Cu) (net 1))
 (segment (start 22.36 -13.2) (end 24.63 -15.47) (width 0.25) (layer F.Cu) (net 1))
 (segment (start 82.13245 -15.47) (end 85.023032 -18.360582) (width 0.25) (layer F.Cu) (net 1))
 (segment (start 22.36 -13.19) (end 22.36 -13.2) (width 0.25) (layer F.Cu) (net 1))
 (segment (start 20.02467 3.626726) (end 21.730334 1.921062) (width 0.25) (layer F.Cu) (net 1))
 (segment (start 15.624747 -12.794013) (end 17.77876 -10.64) (width 0.25) (layer F.Cu) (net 1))
 (segment (start 19.81 -10.64) (end 20.855 -11.685) (width 0.25) (layer F.Cu) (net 1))
 (segment (start 20.855 -11.685) (end 22.36 -13.19) (width 0.25) (layer F.Cu) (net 1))
 (segment (start 20.595531 -11.425531) (end 20.855 -11.685) (width 0.25) (layer F.Cu) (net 1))
 (segment (start 23.971518 -16.208482) (end 24.71 -15.47) (width 0.25) (layer F.Cu) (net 1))
 (segment (start 23.971518 -20.246421) (end 23.971518 -16.208482) (width 0.25) (layer F.Cu) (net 1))
 (segment (start 24.63 -15.47) (end 24.71 -15.47) (width 0.25) (layer F.Cu) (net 1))
 (segment (start 35.060931 -21.044767) (end 41.943412 -27.927248) (width 0.25) (layer F.Cu) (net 1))
 (segment (start 33.096661 -21.044767) (end 35.060931 -21.044767) (width 0.25) (layer F.Cu) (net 1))
 (segment (start 56.770078 -22.260582) (end 51.103412 -27.927248) (width 0.25) (layer F.Cu) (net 1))
 (segment (start 59.943413 -22.260582) (end 56.770078 -22.260582) (width 0.25) (layer F.Cu) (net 1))
 (segment (start 56.770078 -39.260582) (end 51.103412 -44.927248) (width 0.25) (layer F.Cu) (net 1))
 (segment (start 59.943412 -39.260582) (end 56.770078 -39.260582) (width 0.25) (layer F.Cu) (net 1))
 (segment (start 31.615013 -37.980076) (end 34.99624 -37.980076) (width 0.25) (layer F.Cu) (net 1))
 (segment (start 22.48987 -37.18173) (end 19.96 -34.65186) (width 0.25) (layer F.Cu) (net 1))
 (segment (start 19.96 -24.257939) (end 23.971518 -20.246421) (width 0.25) (layer F.Cu) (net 1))
 (segment (start 19.96 -34.65186) (end 19.96 -24.257939) (width 0.25) (layer F.Cu) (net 1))
 (segment (start 37.063082 -32.807578) (end 41.943412 -27.927248) (width 0.25) (layer F.Cu) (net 1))
 (segment (start 37.063082 -40.046918) (end 37.063082 -32.807578) (width 0.25) (layer F.Cu) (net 1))
 (segment (start 34.99624 -37.980076) (end 37.063082 -40.046918) (width 0.25) (layer F.Cu) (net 1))
 (segment (start 37.063082 -40.046918) (end 41.943412 -44.927248) (width 0.25) (layer F.Cu) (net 1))
 (segment (start 56.770078 -25.433917) (end 59.943413 -22.260582) (width 0.25) (layer F.Cu) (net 1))
 (segment (start 56.770078 -39.260582) (end 56.770078 -25.433917) (width 0.25) (layer F.Cu) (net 1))
 (segment (start 41.943412 -18.036588) (end 44.51 -15.47) (width 0.25) (layer F.Cu) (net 1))
 (segment (start 41.943412 -27.927248) (end 41.943412 -18.036588) (width 0.25) (layer F.Cu) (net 1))
 (segment (start 24.71 -15.47) (end 44.51 -15.47) (width 0.25) (layer F.Cu) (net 1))
 (segment (start 59.943413 -18.016587) (end 62.49 -15.47) (width 0.25) (layer F.Cu) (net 1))
 (segment (start 59.943413 -22.260582) (end 59.943413 -18.016587) (width 0.25) (layer F.Cu) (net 1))
 (segment (start 62.49 -15.47) (end 82.13245 -15.47) (width 0.25) (layer F.Cu) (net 1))
 (segment (start 44.51 -15.47) (end 62.49 -15.47) (width 0.25) (layer F.Cu) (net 1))
 (segment (start 78.939419 -46.290581) (end 77.903412 -46.290581) (width 0.25) (layer F.Cu) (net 1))
 (segment (start 86.023792 -39.206208) (end 78.939419 -46.290581) (width 0.25) (layer F.Cu) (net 1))
 (segment (start 86.023792 -18.360582) (end 86.023792 -39.206208) (width 0.25) (layer F.Cu) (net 1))
 (segment (start 21.730334 1.921062) (end 18.73 -10.64) (width 0.25) (layer F.Cu) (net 1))
 (segment (start 18.73 -10.64) (end 19.81 -10.64) (width 0.25) (layer F.Cu) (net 1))
 (segment (start 17.77876 -10.64) (end 18.73 -10.64) (width 0.25) (layer F.Cu) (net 1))
 (segment (start 13.746524 5.619534) (end 17.610228 4.584257) (width 0.25) (layer B.Cu) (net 2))
 (segment (start 76.366415 -19.353585) (end 77.903412 -20.890581) (width 0.25) (layer B.Cu) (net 2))
 (segment (start 18.24597 5.22) (end 20.61 5.22) (width 0.25) (layer B.Cu) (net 2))
 (segment (start 17.610227 4.584257) (end 18.24597 5.22) (width 0.25) (layer B.Cu) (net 2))
 (segment (start 20.595531 -11.415531) (end 24.65 -15.47) (width 0.25) (layer B.Cu) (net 2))
 (segment (start 20.61 5.22) (end 21.79 4.04) (width 0.25) (layer B.Cu) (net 2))
 (segment (start 76.366415 -17.126415) (end 76.366415 -19.353585) (width 0.25) (layer B.Cu) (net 2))
 (segment (start 24.65 -15.47) (end 74.71 -15.47) (width 0.25) (layer B.Cu) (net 2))
 (segment (start 74.71 -15.47) (end 76.366415 -17.126415) (width 0.25) (layer B.Cu) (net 2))
 (segment (start 21.79 4.04) (end 21.79 1.97) (width 0.25) (layer B.Cu) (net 2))
 (segment (start 20.595531 -11.415531) (end 18.941011 -9.751011) (width 0.25) (layer B.Cu) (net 2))
 (segment (start 21.79 1.97) (end 18.941011 -9.751011) (width 0.25) (layer B.Cu) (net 2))
 (segment (start 9.346602 -10.801206) (end 13.210305 -11.836482) (width 0.25) (layer B.Cu) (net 3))
 (segment (start 13.210304 -11.836482) (end 14.066786 -10.98) (width 0.25) (layer B.Cu) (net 3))
 (segment (start 19.52359 -10.98) (end 24.4636 -15.92001) (width 0.25) (layer B.Cu) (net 3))
 (segment (start 14.066786 -10.98) (end 19.52359 -10.98) (width 0.25) (layer B.Cu) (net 3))
 (segment (start 24.4636 -15.92001) (end 74.5236 -15.92001) (width 0.25) (layer B.Cu) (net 3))
 (segment (start 75.916405 -21.443574) (end 77.903412 -23.430581) (width 0.25) (layer B.Cu) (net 3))
 (segment (start 75.916405 -17.312815) (end 75.916405 -21.443574) (width 0.25) (layer B.Cu) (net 3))
 (segment (start 74.5236 -15.92001) (end 75.916405 -17.312815) (width 0.25) (layer B.Cu) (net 3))
 (segment (start 26.567847 -20.172423) (end 30.552625 -20.521047) (width 0.25) (layer B.Cu) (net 4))
 (segment (start 30.552625 -20.521047) (end 30.552625 -17.137395) (width 0.25) (layer B.Cu) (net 4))
 (segment (start 30.552625 -17.137395) (end 31.32 -16.37002) (width 0.25) (layer B.Cu) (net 4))
 (segment (start 31.32 -16.37002) (end 74.3372 -16.37002) (width 0.25) (layer B.Cu) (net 4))
 (segment (start 75.466395 -23.533564) (end 77.903412 -25.970581) (width 0.25) (layer B.Cu) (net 4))
 (segment (start 75.466395 -17.499215) (end 75.466395 -23.533564) (width 0.25) (layer B.Cu) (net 4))
 (segment (start 74.3372 -16.37002) (end 75.466395 -17.499215) (width 0.25) (layer B.Cu) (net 4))
 (segment (start 25.086199 -37.107732) (end 29.070978 -37.456355) (width 0.25) (layer B.Cu) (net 5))
 (segment (start 29.070977 -37.456356) (end 35.67 -30.857333) (width 0.25) (layer B.Cu) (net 5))
 (segment (start 35.67 -17.53) (end 36.37997 -16.82003) (width 0.25) (layer B.Cu) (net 5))
 (segment (start 35.67 -30.857333) (end 35.67 -17.53) (width 0.25) (layer B.Cu) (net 5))
 (segment (start 36.37997 -16.82003) (end 74.1508 -16.82003) (width 0.25) (layer B.Cu) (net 5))
 (segment (start 75.016385 -25.623554) (end 77.903412 -28.510581) (width 0.25) (layer B.Cu) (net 5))
 (segment (start 75.016385 -17.685615) (end 75.016385 -25.623554) (width 0.25) (layer B.Cu) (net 5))
 (segment (start 74.1508 -16.82003) (end 75.016385 -17.685615) (width 0.25) (layer B.Cu) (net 5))
 (segment (start 44.523412 -27.627247) (end 48.523412 -27.627248) (width 0.25) (layer B.Cu) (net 6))
 (segment (start 48.523412 -27.627248) (end 48.523412 -18.056628) (width 0.25) (layer B.Cu) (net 6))
 (segment (start 48.523412 -18.056628) (end 49.31 -17.27004) (width 0.25) (layer B.Cu) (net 6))
 (segment (start 49.31 -17.27004) (end 73.9644 -17.27004) (width 0.25) (layer B.Cu) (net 6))
 (segment (start 73.9644 -17.27004) (end 74.566375 -17.872015) (width 0.25) (layer B.Cu) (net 6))
 (segment (start 74.566375 -27.713544) (end 77.903412 -31.050581) (width 0.25) (layer B.Cu) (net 6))
 (segment (start 74.566375 -17.872015) (end 74.566375 -27.713544) (width 0.25) (layer B.Cu) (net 6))
 (segment (start 44.523411 -44.627247) (end 48.523412 -44.627248) (width 0.25) (layer B.Cu) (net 7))
 (segment (start 48.523412 -44.627248) (end 54.61066 -38.54) (width 0.25) (layer B.Cu) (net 7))
 (segment (start 54.61066 -18.36934) (end 55.25995 -17.72005) (width 0.25) (layer B.Cu) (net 7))
 (segment (start 54.61066 -38.54) (end 54.61066 -18.36934) (width 0.25) (layer B.Cu) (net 7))
 (segment (start 55.25995 -17.72005) (end 73.778 -17.72005) (width 0.25) (layer B.Cu) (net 7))
 (segment (start 73.778 -17.72005) (end 74.116365 -18.058415) (width 0.25) (layer B.Cu) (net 7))
 (segment (start 74.116365 -29.803534) (end 74.116365 -28.636365) (width 0.25) (layer B.Cu) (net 7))
 (segment (start 77.903412 -33.590581) (end 74.116365 -29.803534) (width 0.25) (layer B.Cu) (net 7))
 (segment (start 74.116365 -28.636365) (end 74.116365 -29.04146) (width 0.25) (layer B.Cu) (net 7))
 (segment (start 74.116365 -18.058415) (end 74.116365 -28.636365) (width 0.25) (layer B.Cu) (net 7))
 (segment (start 62.523412 -21.960583) (end 66.523412 -21.960582) (width 0.25) (layer B.Cu) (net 8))
 (segment (start 66.523413 -21.960582) (end 66.523413 -18.696647) (width 0.25) (layer B.Cu) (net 8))
 (segment (start 66.523413 -18.696647) (end 67.05 -18.17006) (width 0.25) (layer B.Cu) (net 8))
 (segment (start 67.05 -18.17006) (end 73.5916 -18.17006) (width 0.25) (layer B.Cu) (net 8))
 (segment (start 73.5916 -18.17006) (end 73.666355 -18.244815) (width 0.25) (layer B.Cu) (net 8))
 (segment (start 77.903412 -36.130581) (end 73.666355 -31.893524) (width 0.25) (layer B.Cu) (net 8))
 (segment (start 73.666355 -28.796355) (end 73.666356 -29.989935) (width 0.25) (layer B.Cu) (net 8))
 (segment (start 73.666355 -31.893524) (end 73.666355 -28.796355) (width 0.25) (layer B.Cu) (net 8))
 (segment (start 73.666355 -18.244815) (end 73.666355 -28.796355) (width 0.25) (layer B.Cu) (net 8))
 (segment (start 62.523412 -38.960581) (end 66.523411 -38.960581) (width 0.25) (layer B.Cu) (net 9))
 (segment (start 66.523412 -38.960582) (end 68.833994 -36.65) (width 0.25) (layer B.Cu) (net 9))
 (segment (start 75.882831 -36.65) (end 77.903412 -38.670581) (width 0.25) (layer B.Cu) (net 9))
 (segment (start 68.833994 -36.65) (end 75.882831 -36.65) (width 0.25) (layer B.Cu) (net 9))
 (segment (start 97.193937 -1.662221) (end 101.05764 -0.626944) (width 0.25) (layer B.Cu) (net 10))
 (segment (start 97.193938 -1.66222) (end 96.431718 -0.9) (width 0.25) (layer B.Cu) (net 10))
 (segment (start 96.431718 -0.9) (end 93.01 -0.9) (width 0.25) (layer B.Cu) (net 10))
 (segment (start 93.01 -0.9) (end 89.97 -3.94) (width 0.25) (layer B.Cu) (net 10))
 (segment (start 89.97 -17.717169) (end 93.143412 -20.890581) (width 0.25) (layer B.Cu) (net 10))
 (segment (start 89.97 -3.94) (end 89.97 -17.717169) (width 0.25) (layer B.Cu) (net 10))
 (segment (start 86.023792 -39.170961) (end 93.143412 -46.290581) (width 0.25) (layer B.Cu) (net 15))
 (segment (start 86.023792 -18.360582) (end 86.023792 -39.170961) (width 0.25) (layer B.Cu) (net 15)))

